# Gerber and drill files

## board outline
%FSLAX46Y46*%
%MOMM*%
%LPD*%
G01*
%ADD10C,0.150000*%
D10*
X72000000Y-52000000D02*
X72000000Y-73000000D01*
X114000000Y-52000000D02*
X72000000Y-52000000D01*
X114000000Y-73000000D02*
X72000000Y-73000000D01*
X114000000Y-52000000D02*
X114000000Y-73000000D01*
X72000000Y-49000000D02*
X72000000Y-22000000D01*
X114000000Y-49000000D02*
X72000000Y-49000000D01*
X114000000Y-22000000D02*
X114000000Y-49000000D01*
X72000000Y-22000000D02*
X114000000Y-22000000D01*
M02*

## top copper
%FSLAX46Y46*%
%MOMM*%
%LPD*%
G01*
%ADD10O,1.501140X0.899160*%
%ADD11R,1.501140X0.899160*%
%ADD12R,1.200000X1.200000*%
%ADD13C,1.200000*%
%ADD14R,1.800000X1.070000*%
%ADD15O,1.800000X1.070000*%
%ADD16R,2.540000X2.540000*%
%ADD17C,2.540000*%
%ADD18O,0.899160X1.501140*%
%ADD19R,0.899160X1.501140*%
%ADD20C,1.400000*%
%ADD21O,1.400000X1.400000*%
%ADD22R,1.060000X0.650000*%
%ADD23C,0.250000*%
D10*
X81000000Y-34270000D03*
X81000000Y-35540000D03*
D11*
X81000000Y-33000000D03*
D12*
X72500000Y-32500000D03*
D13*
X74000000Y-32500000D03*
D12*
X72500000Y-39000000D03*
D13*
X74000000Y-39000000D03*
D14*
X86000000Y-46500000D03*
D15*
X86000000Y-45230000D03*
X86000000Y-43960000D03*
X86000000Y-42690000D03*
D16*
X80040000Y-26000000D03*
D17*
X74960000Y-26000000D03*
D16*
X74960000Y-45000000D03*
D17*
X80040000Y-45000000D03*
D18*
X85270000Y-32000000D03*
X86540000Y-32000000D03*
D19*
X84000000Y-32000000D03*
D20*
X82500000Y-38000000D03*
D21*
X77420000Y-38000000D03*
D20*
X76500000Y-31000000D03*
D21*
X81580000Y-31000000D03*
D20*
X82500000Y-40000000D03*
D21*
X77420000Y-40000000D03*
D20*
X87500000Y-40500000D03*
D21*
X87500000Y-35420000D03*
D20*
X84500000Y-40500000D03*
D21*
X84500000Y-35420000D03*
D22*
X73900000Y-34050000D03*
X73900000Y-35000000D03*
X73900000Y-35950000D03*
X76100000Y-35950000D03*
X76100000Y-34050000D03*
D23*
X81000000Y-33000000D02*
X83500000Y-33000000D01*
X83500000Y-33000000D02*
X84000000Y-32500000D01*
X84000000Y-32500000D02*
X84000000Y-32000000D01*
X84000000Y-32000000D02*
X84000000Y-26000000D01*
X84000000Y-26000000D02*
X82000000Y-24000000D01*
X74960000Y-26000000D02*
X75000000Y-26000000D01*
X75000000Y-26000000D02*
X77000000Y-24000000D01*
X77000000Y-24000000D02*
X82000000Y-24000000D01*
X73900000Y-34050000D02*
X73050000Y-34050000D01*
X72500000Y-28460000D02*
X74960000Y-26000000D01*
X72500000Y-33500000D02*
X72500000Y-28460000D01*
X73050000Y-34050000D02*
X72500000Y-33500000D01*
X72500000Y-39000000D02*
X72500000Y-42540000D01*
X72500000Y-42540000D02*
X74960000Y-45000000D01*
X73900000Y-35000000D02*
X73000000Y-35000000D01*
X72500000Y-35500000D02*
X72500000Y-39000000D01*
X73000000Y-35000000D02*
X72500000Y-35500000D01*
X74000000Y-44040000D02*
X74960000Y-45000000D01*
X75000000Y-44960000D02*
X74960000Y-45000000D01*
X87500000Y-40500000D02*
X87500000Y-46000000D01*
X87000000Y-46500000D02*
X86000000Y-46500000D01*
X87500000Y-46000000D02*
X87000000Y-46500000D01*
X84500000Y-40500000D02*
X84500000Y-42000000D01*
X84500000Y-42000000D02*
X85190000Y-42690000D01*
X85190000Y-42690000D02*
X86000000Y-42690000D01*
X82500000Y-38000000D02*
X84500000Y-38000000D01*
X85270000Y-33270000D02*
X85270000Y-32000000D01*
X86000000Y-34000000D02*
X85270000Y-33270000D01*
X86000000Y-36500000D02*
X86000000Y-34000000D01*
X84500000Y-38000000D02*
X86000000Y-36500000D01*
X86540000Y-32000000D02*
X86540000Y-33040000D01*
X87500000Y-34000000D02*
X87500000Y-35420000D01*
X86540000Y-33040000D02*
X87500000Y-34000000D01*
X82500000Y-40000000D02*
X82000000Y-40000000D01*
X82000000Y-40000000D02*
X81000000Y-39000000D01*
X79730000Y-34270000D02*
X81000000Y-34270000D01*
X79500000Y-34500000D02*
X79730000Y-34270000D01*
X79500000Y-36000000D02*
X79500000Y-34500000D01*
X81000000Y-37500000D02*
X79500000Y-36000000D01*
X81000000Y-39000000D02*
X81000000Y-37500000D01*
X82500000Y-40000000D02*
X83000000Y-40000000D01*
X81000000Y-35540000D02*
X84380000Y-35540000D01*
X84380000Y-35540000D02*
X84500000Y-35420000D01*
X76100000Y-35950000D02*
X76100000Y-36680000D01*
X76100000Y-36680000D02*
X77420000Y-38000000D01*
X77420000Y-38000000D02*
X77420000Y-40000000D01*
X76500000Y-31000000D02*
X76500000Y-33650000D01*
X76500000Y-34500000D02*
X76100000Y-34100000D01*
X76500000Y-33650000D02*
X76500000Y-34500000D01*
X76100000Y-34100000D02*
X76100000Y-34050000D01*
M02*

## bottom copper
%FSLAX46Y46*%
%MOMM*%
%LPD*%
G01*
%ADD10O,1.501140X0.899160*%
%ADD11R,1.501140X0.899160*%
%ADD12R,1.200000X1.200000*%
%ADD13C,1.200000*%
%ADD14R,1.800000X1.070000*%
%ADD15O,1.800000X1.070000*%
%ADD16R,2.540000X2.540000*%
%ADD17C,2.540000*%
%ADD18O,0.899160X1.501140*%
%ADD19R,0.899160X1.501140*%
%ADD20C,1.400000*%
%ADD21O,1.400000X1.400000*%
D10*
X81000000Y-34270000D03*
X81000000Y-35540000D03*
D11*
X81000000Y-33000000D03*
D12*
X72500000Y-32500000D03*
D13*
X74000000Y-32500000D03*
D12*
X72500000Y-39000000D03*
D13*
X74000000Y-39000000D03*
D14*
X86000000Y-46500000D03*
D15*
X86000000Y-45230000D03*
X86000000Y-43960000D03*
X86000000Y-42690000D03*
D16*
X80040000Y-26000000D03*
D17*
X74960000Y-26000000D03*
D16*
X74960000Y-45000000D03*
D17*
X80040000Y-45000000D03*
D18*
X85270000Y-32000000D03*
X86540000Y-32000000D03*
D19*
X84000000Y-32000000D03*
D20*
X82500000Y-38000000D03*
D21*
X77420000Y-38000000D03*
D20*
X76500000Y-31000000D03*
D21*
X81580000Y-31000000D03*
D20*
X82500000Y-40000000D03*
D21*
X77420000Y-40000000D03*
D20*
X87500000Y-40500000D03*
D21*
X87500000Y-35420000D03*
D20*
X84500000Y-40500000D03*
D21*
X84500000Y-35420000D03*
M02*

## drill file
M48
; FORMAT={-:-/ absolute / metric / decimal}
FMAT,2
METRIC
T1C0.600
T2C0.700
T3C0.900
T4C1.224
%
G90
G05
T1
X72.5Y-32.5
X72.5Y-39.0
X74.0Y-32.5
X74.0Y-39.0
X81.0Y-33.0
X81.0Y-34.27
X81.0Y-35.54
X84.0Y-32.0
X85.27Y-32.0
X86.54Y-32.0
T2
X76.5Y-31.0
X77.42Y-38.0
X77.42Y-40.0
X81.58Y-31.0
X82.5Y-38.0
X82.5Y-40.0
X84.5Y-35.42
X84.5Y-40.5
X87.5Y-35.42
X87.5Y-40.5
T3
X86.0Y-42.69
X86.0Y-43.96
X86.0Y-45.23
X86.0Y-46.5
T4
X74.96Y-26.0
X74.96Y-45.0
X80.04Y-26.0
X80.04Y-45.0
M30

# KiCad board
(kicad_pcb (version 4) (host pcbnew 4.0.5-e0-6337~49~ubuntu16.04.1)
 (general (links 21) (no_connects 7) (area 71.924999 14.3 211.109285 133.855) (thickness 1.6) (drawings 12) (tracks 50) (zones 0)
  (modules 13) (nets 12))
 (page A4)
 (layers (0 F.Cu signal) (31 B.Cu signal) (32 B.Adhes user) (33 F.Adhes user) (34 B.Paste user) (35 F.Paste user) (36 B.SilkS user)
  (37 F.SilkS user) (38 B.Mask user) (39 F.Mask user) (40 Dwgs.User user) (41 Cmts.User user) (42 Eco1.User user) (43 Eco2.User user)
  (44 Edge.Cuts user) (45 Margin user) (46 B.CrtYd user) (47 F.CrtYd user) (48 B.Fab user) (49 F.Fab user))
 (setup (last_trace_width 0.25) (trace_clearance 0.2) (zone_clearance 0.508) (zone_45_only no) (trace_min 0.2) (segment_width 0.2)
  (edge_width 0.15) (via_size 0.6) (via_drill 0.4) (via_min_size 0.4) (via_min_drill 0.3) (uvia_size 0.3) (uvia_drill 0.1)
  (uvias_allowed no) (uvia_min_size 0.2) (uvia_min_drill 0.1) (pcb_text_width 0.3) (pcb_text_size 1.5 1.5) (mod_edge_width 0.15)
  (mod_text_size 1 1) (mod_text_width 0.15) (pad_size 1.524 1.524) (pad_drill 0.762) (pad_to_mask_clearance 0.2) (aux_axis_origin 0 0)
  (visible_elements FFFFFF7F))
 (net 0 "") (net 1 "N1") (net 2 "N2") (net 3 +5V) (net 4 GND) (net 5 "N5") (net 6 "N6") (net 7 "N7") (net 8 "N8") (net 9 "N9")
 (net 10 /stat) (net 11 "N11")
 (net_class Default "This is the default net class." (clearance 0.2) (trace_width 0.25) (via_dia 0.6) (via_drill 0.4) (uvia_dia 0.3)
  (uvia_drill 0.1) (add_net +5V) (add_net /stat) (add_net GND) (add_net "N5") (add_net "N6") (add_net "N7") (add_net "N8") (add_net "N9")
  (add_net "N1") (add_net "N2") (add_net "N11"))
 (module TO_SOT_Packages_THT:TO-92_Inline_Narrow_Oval (layer F.Cu) (at 81 33 270)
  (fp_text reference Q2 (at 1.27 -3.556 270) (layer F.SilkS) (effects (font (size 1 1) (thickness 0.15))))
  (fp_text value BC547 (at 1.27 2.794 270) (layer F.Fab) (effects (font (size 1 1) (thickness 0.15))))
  (pad 2 thru_hole oval (at 1.27 0 90) (size 0.89916 1.50114) (drill 0.6) (layers *.Cu *.Mask) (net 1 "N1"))
  (pad 3 thru_hole oval (at 2.54 0 90) (size 0.89916 1.50114) (drill 0.6) (layers *.Cu *.Mask) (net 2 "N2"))
  (pad 1 thru_hole rect (at 0 0 90) (size 0.89916 1.50114) (drill 0.6) (layers *.Cu *.Mask) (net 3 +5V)))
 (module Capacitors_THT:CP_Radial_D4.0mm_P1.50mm (layer F.Cu) (at 72.5 32.5)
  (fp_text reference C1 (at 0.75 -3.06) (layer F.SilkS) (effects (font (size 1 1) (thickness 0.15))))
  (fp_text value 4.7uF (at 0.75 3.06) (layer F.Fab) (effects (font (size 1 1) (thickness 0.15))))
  (pad 1 thru_hole rect (at 0 0) (size 1.2 1.2) (drill 0.6) (layers *.Cu *.Mask) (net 3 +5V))
  (pad 2 thru_hole circle (at 1.5 0) (size 1.2 1.2) (drill 0.6) (layers *.Cu *.Mask) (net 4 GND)))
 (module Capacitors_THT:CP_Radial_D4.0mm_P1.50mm (layer F.Cu) (at 72.5 39)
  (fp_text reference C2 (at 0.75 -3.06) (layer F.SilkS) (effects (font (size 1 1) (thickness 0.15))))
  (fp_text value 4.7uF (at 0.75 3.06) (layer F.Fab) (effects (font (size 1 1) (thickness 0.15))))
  (pad 1 thru_hole rect (at 0 0) (size 1.2 1.2) (drill 0.6) (layers *.Cu *.Mask) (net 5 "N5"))
  (pad 2 thru_hole circle (at 1.5 0) (size 1.2 1.2) (drill 0.6) (layers *.Cu *.Mask) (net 4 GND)))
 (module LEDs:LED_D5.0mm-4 (layer F.Cu) (at 86 46.5 90)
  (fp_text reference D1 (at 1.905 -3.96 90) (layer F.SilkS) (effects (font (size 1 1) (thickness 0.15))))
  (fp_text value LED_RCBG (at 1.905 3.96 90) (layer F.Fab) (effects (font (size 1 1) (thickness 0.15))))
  (pad 1 thru_hole rect (at 0 0 90) (size 1.07 1.8) (drill 0.9) (layers *.Cu *.Mask) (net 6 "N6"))
  (pad 2 thru_hole oval (at 1.27 0 90) (size 1.07 1.8) (drill 0.9) (layers *.Cu *.Mask) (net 4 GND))
  (pad 3 thru_hole oval (at 2.54 0 90) (size 1.07 1.8) (drill 0.9) (layers *.Cu *.Mask))
  (pad 4 thru_hole oval (at 3.81 0 90) (size 1.07 1.8) (drill 0.9) (layers *.Cu *.Mask) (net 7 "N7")))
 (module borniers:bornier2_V (layer F.Cu) (at 77.5 26 180)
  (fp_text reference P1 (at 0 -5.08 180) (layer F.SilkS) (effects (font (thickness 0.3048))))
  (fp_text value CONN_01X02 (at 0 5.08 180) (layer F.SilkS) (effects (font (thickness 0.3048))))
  (pad 1 thru_hole rect (at -2.54 0 180) (size 2.54 2.54) (drill 1.22428) (layers *.Cu *.Mask F.SilkS) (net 4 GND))
  (pad 2 thru_hole circle (at 2.54 0 180) (size 2.54 2.54) (drill 1.22428) (layers *.Cu *.Mask F.SilkS) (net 3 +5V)))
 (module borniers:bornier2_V (layer F.Cu) (at 77.5 45)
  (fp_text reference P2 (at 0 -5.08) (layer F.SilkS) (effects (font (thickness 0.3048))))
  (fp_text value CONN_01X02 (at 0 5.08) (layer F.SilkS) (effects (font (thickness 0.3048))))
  (pad 1 thru_hole rect (at -2.54 0) (size 2.54 2.54) (drill 1.22428) (layers *.Cu *.Mask F.SilkS) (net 5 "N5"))
  (pad 2 thru_hole circle (at 2.54 0) (size 2.54 2.54) (drill 1.22428) (layers *.Cu *.Mask F.SilkS) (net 4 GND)))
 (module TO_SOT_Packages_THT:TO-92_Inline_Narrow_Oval (layer F.Cu) (at 84 32)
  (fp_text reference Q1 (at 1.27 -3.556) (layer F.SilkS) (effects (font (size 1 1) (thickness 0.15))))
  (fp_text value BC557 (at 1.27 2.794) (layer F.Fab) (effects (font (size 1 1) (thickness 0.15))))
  (pad 2 thru_hole oval (at 1.27 0 180) (size 0.89916 1.50114) (drill 0.6) (layers *.Cu *.Mask) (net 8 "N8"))
  (pad 3 thru_hole oval (at 2.54 0 180) (size 0.89916 1.50114) (drill 0.6) (layers *.Cu *.Mask) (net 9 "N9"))
  (pad 1 thru_hole rect (at 0 0 180) (size 0.89916 1.50114) (drill 0.6) (layers *.Cu *.Mask) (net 3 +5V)))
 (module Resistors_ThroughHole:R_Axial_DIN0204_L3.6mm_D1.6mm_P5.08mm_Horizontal (layer F.Cu) (at 82.5 38 180)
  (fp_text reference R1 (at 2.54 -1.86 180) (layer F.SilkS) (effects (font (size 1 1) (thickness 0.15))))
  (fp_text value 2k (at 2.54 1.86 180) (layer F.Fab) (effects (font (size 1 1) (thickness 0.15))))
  (pad 1 thru_hole circle (at 0 0 180) (size 1.4 1.4) (drill 0.7) (layers *.Cu *.Mask) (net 8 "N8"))
  (pad 2 thru_hole oval (at 5.08 0 180) (size 1.4 1.4) (drill 0.7) (layers *.Cu *.Mask) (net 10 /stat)))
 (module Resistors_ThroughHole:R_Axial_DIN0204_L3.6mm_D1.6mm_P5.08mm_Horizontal (layer F.Cu) (at 76.5 31)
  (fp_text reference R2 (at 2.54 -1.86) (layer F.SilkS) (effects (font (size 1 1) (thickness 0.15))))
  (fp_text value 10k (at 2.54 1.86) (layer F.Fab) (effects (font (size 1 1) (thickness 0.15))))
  (pad 1 thru_hole circle (at 0 0) (size 1.4 1.4) (drill 0.7) (layers *.Cu *.Mask) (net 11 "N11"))
  (pad 2 thru_hole oval (at 5.08 0) (size 1.4 1.4) (drill 0.7) (layers *.Cu *.Mask) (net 4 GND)))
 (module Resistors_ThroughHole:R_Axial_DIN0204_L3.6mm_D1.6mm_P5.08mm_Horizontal (layer F.Cu) (at 82.5 40 180)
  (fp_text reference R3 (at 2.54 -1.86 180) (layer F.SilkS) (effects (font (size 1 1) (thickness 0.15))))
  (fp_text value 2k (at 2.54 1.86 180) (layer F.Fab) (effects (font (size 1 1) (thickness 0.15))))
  (pad 1 thru_hole circle (at 0 0 180) (size 1.4 1.4) (drill 0.7) (layers *.Cu *.Mask) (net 1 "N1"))
  (pad 2 thru_hole oval (at 5.08 0 180) (size 1.4 1.4) (drill 0.7) (layers *.Cu *.Mask) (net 10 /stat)))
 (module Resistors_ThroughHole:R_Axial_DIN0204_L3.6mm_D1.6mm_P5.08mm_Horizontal (layer F.Cu) (at 87.5 40.5 90)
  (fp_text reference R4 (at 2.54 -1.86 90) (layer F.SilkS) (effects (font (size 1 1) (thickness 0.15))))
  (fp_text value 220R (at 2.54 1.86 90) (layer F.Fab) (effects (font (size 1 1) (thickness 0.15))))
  (pad 1 thru_hole circle (at 0 0 90) (size 1.4 1.4) (drill 0.7) (layers *.Cu *.Mask) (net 6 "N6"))
  (pad 2 thru_hole oval (at 5.08 0 90) (size 1.4 1.4) (drill 0.7) (layers *.Cu *.Mask) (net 9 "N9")))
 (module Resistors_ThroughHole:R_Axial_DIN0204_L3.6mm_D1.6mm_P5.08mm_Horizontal (layer F.Cu) (at 84.5 40.5 90)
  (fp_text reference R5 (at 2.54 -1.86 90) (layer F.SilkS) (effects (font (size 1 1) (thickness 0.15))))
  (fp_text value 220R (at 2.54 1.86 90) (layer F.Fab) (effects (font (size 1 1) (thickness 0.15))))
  (pad 1 thru_hole circle (at 0 0 90) (size 1.4 1.4) (drill 0.7) (layers *.Cu *.Mask) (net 7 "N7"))
  (pad 2 thru_hole oval (at 5.08 0 90) (size 1.4 1.4) (drill 0.7) (layers *.Cu *.Mask) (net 2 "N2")))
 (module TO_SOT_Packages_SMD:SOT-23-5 (layer F.Cu) (at 75 35)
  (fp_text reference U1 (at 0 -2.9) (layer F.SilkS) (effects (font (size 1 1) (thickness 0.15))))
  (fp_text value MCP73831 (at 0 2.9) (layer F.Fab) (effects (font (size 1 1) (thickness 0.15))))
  (pad 1 smd rect (at -1.1 -0.95) (size 1.06 0.65) (layers F.Cu F.Paste F.Mask) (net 3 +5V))
  (pad 2 smd rect (at -1.1 0) (size 1.06 0.65) (layers F.Cu F.Paste F.Mask) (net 5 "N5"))
  (pad 3 smd rect (at -1.1 0.95) (size 1.06 0.65) (layers F.Cu F.Paste F.Mask) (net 4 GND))
  (pad 4 smd rect (at 1.1 0.95) (size 1.06 0.65) (layers F.Cu F.Paste F.Mask) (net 10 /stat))
  (pad 5 smd rect (at 1.1 -0.95) (size 1.06 0.65) (layers F.Cu F.Paste F.Mask) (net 11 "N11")))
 (gr_line (start 72 52) (end 72 73) (angle 90) (layer Edge.Cuts) (width 0.15))
 (gr_line (start 114 52) (end 72 52) (angle 90) (layer Edge.Cuts) (width 0.15))
 (gr_line (start 114 73) (end 72 73) (angle 90) (layer Edge.Cuts) (width 0.15))
 (gr_line (start 114 52) (end 114 73) (angle 90) (layer Edge.Cuts) (width 0.15))
 (gr_line (start 72 49) (end 72 22) (angle 90) (layer Edge.Cuts) (width 0.15))
 (gr_line (start 114 49) (end 72 49) (angle 90) (layer Edge.Cuts) (width 0.15))
 (gr_line (start 114 22) (end 114 49) (angle 90) (layer Edge.Cuts) (width 0.15))
 (gr_line (start 72 22) (end 114 22) (angle 90) (layer Edge.Cuts) (width 0.15))
 (segment (start 81 33) (end 83.5 33) (width 0.25) (layer F.Cu) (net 3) (status 400000))
 (segment (start 83.5 33) (end 84 32.5) (width 0.25) (layer F.Cu) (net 3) (status 800000))
 (segment (start 84 32.5) (end 84 32) (width 0.25) (layer F.Cu) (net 3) (status C00000))
 (segment (start 84 32) (end 84 26) (width 0.25) (layer F.Cu) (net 3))
 (segment (start 84 26) (end 82 24) (width 0.25) (layer F.Cu) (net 3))
 (segment (start 74.96 26) (end 75 26) (width 0.25) (layer F.Cu) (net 3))
 (segment (start 75 26) (end 77 24) (width 0.25) (layer F.Cu) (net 3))
 (segment (start 77 24) (end 82 24) (width 0.25) (layer F.Cu) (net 3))
 (segment (start 73.9 34.05) (end 73.05 34.05) (width 0.25) (layer F.Cu) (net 3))
 (segment (start 72.5 28.46) (end 74.96 26) (width 0.25) (layer F.Cu) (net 3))
 (segment (start 72.5 33.5) (end 72.5 28.46) (width 0.25) (layer F.Cu) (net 3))
 (segment (start 73.05 34.05) (end 72.5 33.5) (width 0.25) (layer F.Cu) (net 3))
 (segment (start 72.5 39) (end 72.5 42.54) (width 0.25) (layer F.Cu) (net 5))
 (segment (start 72.5 42.54) (end 74.96 45) (width 0.25) (layer F.Cu) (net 5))
 (segment (start 73.9 35) (end 73 35) (width 0.25) (layer F.Cu) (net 5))
 (segment (start 72.5 35.5) (end 72.5 39) (width 0.25) (layer F.Cu) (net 5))
 (segment (start 73 35) (end 72.5 35.5) (width 0.25) (layer F.Cu) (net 5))
 (segment (start 74 44.04) (end 74.96 45) (width 0.25) (layer F.Cu) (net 5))
 (segment (start 75 44.96) (end 74.96 45) (width 0.25) (layer F.Cu) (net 5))
 (segment (start 87.5 40.5) (end 87.5 46) (width 0.25) (layer F.Cu) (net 6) (status 400000))
 (segment (start 87 46.5) (end 86 46.5) (width 0.25) (layer F.Cu) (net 6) (status 800000))
 (segment (start 87.5 46) (end 87 46.5) (width 0.25) (layer F.Cu) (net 6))
 (segment (start 84.5 40.5) (end 84.5 42) (width 0.25) (layer F.Cu) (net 7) (status 400000))
 (segment (start 84.5 42) (end 85.19 42.69) (width 0.25) (layer F.Cu) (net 7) (status 800000))
 (segment (start 85.19 42.69) (end 86 42.69) (width 0.25) (layer F.Cu) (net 7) (status C00000))
 (segment (start 82.5 38) (end 84.5 38) (width 0.25) (layer F.Cu) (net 8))
 (segment (start 85.27 33.27) (end 85.27 32) (width 0.25) (layer F.Cu) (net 8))
 (segment (start 86 34) (end 85.27 33.27) (width 0.25) (layer F.Cu) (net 8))
 (segment (start 86 36.5) (end 86 34) (width 0.25) (layer F.Cu) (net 8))
 (segment (start 84.5 38) (end 86 36.5) (width 0.25) (layer F.Cu) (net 8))
 (segment (start 86.54 32) (end 86.54 33.04) (width 0.25) (layer F.Cu) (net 9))
 (segment (start 87.5 34) (end 87.5 35.42) (width 0.25) (layer F.Cu) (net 9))
 (segment (start 86.54 33.04) (end 87.5 34) (width 0.25) (layer F.Cu) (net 9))
 (segment (start 82.5 40) (end 82 40) (width 0.25) (layer F.Cu) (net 1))
 (segment (start 82 40) (end 81 39) (width 0.25) (layer F.Cu) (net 1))
 (segment (start 79.73 34.27) (end 81 34.27) (width 0.25) (layer F.Cu) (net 1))
 (segment (start 79.5 34.5) (end 79.73 34.27) (width 0.25) (layer F.Cu) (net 1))
 (segment (start 79.5 36) (end 79.5 34.5) (width 0.25) (layer F.Cu) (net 1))
 (segment (start 81 37.5) (end 79.5 36) (width 0.25) (layer F.Cu) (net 1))
 (segment (start 81 39) (end 81 37.5) (width 0.25) (layer F.Cu) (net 1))
 (segment (start 82.5 40) (end 83 40) (width 0.25) (layer F.Cu) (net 1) (status 30))
 (segment (start 81 35.54) (end 84.38 35.54) (width 0.25) (layer F.Cu) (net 2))
 (segment (start 84.38 35.54) (end 84.5 35.42) (width 0.25) (layer F.Cu) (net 2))
 (segment (start 76.1 35.95) (end 76.1 36.68) (width 0.25) (layer F.Cu) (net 10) (status 400000))
 (segment (start 76.1 36.68) (end 77.42 38) (width 0.25) (layer F.Cu) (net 10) (status 800000))
 (segment (start 77.42 38) (end 77.42 40) (width 0.25) (layer F.Cu) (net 10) (status 20))
 (segment (start 76.5 31) (end 76.5 33.65) (width 0.25) (layer F.Cu) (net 11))
 (segment (start 76.5 34.5) (end 76.1 34.1) (width 0.25) (layer F.Cu) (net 11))
 (segment (start 76.5 33.65) (end 76.5 34.5) (width 0.25) (layer F.Cu) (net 11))
 (segment (start 76.1 34.1) (end 76.1 34.05) (width 0.25) (layer F.Cu) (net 11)))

